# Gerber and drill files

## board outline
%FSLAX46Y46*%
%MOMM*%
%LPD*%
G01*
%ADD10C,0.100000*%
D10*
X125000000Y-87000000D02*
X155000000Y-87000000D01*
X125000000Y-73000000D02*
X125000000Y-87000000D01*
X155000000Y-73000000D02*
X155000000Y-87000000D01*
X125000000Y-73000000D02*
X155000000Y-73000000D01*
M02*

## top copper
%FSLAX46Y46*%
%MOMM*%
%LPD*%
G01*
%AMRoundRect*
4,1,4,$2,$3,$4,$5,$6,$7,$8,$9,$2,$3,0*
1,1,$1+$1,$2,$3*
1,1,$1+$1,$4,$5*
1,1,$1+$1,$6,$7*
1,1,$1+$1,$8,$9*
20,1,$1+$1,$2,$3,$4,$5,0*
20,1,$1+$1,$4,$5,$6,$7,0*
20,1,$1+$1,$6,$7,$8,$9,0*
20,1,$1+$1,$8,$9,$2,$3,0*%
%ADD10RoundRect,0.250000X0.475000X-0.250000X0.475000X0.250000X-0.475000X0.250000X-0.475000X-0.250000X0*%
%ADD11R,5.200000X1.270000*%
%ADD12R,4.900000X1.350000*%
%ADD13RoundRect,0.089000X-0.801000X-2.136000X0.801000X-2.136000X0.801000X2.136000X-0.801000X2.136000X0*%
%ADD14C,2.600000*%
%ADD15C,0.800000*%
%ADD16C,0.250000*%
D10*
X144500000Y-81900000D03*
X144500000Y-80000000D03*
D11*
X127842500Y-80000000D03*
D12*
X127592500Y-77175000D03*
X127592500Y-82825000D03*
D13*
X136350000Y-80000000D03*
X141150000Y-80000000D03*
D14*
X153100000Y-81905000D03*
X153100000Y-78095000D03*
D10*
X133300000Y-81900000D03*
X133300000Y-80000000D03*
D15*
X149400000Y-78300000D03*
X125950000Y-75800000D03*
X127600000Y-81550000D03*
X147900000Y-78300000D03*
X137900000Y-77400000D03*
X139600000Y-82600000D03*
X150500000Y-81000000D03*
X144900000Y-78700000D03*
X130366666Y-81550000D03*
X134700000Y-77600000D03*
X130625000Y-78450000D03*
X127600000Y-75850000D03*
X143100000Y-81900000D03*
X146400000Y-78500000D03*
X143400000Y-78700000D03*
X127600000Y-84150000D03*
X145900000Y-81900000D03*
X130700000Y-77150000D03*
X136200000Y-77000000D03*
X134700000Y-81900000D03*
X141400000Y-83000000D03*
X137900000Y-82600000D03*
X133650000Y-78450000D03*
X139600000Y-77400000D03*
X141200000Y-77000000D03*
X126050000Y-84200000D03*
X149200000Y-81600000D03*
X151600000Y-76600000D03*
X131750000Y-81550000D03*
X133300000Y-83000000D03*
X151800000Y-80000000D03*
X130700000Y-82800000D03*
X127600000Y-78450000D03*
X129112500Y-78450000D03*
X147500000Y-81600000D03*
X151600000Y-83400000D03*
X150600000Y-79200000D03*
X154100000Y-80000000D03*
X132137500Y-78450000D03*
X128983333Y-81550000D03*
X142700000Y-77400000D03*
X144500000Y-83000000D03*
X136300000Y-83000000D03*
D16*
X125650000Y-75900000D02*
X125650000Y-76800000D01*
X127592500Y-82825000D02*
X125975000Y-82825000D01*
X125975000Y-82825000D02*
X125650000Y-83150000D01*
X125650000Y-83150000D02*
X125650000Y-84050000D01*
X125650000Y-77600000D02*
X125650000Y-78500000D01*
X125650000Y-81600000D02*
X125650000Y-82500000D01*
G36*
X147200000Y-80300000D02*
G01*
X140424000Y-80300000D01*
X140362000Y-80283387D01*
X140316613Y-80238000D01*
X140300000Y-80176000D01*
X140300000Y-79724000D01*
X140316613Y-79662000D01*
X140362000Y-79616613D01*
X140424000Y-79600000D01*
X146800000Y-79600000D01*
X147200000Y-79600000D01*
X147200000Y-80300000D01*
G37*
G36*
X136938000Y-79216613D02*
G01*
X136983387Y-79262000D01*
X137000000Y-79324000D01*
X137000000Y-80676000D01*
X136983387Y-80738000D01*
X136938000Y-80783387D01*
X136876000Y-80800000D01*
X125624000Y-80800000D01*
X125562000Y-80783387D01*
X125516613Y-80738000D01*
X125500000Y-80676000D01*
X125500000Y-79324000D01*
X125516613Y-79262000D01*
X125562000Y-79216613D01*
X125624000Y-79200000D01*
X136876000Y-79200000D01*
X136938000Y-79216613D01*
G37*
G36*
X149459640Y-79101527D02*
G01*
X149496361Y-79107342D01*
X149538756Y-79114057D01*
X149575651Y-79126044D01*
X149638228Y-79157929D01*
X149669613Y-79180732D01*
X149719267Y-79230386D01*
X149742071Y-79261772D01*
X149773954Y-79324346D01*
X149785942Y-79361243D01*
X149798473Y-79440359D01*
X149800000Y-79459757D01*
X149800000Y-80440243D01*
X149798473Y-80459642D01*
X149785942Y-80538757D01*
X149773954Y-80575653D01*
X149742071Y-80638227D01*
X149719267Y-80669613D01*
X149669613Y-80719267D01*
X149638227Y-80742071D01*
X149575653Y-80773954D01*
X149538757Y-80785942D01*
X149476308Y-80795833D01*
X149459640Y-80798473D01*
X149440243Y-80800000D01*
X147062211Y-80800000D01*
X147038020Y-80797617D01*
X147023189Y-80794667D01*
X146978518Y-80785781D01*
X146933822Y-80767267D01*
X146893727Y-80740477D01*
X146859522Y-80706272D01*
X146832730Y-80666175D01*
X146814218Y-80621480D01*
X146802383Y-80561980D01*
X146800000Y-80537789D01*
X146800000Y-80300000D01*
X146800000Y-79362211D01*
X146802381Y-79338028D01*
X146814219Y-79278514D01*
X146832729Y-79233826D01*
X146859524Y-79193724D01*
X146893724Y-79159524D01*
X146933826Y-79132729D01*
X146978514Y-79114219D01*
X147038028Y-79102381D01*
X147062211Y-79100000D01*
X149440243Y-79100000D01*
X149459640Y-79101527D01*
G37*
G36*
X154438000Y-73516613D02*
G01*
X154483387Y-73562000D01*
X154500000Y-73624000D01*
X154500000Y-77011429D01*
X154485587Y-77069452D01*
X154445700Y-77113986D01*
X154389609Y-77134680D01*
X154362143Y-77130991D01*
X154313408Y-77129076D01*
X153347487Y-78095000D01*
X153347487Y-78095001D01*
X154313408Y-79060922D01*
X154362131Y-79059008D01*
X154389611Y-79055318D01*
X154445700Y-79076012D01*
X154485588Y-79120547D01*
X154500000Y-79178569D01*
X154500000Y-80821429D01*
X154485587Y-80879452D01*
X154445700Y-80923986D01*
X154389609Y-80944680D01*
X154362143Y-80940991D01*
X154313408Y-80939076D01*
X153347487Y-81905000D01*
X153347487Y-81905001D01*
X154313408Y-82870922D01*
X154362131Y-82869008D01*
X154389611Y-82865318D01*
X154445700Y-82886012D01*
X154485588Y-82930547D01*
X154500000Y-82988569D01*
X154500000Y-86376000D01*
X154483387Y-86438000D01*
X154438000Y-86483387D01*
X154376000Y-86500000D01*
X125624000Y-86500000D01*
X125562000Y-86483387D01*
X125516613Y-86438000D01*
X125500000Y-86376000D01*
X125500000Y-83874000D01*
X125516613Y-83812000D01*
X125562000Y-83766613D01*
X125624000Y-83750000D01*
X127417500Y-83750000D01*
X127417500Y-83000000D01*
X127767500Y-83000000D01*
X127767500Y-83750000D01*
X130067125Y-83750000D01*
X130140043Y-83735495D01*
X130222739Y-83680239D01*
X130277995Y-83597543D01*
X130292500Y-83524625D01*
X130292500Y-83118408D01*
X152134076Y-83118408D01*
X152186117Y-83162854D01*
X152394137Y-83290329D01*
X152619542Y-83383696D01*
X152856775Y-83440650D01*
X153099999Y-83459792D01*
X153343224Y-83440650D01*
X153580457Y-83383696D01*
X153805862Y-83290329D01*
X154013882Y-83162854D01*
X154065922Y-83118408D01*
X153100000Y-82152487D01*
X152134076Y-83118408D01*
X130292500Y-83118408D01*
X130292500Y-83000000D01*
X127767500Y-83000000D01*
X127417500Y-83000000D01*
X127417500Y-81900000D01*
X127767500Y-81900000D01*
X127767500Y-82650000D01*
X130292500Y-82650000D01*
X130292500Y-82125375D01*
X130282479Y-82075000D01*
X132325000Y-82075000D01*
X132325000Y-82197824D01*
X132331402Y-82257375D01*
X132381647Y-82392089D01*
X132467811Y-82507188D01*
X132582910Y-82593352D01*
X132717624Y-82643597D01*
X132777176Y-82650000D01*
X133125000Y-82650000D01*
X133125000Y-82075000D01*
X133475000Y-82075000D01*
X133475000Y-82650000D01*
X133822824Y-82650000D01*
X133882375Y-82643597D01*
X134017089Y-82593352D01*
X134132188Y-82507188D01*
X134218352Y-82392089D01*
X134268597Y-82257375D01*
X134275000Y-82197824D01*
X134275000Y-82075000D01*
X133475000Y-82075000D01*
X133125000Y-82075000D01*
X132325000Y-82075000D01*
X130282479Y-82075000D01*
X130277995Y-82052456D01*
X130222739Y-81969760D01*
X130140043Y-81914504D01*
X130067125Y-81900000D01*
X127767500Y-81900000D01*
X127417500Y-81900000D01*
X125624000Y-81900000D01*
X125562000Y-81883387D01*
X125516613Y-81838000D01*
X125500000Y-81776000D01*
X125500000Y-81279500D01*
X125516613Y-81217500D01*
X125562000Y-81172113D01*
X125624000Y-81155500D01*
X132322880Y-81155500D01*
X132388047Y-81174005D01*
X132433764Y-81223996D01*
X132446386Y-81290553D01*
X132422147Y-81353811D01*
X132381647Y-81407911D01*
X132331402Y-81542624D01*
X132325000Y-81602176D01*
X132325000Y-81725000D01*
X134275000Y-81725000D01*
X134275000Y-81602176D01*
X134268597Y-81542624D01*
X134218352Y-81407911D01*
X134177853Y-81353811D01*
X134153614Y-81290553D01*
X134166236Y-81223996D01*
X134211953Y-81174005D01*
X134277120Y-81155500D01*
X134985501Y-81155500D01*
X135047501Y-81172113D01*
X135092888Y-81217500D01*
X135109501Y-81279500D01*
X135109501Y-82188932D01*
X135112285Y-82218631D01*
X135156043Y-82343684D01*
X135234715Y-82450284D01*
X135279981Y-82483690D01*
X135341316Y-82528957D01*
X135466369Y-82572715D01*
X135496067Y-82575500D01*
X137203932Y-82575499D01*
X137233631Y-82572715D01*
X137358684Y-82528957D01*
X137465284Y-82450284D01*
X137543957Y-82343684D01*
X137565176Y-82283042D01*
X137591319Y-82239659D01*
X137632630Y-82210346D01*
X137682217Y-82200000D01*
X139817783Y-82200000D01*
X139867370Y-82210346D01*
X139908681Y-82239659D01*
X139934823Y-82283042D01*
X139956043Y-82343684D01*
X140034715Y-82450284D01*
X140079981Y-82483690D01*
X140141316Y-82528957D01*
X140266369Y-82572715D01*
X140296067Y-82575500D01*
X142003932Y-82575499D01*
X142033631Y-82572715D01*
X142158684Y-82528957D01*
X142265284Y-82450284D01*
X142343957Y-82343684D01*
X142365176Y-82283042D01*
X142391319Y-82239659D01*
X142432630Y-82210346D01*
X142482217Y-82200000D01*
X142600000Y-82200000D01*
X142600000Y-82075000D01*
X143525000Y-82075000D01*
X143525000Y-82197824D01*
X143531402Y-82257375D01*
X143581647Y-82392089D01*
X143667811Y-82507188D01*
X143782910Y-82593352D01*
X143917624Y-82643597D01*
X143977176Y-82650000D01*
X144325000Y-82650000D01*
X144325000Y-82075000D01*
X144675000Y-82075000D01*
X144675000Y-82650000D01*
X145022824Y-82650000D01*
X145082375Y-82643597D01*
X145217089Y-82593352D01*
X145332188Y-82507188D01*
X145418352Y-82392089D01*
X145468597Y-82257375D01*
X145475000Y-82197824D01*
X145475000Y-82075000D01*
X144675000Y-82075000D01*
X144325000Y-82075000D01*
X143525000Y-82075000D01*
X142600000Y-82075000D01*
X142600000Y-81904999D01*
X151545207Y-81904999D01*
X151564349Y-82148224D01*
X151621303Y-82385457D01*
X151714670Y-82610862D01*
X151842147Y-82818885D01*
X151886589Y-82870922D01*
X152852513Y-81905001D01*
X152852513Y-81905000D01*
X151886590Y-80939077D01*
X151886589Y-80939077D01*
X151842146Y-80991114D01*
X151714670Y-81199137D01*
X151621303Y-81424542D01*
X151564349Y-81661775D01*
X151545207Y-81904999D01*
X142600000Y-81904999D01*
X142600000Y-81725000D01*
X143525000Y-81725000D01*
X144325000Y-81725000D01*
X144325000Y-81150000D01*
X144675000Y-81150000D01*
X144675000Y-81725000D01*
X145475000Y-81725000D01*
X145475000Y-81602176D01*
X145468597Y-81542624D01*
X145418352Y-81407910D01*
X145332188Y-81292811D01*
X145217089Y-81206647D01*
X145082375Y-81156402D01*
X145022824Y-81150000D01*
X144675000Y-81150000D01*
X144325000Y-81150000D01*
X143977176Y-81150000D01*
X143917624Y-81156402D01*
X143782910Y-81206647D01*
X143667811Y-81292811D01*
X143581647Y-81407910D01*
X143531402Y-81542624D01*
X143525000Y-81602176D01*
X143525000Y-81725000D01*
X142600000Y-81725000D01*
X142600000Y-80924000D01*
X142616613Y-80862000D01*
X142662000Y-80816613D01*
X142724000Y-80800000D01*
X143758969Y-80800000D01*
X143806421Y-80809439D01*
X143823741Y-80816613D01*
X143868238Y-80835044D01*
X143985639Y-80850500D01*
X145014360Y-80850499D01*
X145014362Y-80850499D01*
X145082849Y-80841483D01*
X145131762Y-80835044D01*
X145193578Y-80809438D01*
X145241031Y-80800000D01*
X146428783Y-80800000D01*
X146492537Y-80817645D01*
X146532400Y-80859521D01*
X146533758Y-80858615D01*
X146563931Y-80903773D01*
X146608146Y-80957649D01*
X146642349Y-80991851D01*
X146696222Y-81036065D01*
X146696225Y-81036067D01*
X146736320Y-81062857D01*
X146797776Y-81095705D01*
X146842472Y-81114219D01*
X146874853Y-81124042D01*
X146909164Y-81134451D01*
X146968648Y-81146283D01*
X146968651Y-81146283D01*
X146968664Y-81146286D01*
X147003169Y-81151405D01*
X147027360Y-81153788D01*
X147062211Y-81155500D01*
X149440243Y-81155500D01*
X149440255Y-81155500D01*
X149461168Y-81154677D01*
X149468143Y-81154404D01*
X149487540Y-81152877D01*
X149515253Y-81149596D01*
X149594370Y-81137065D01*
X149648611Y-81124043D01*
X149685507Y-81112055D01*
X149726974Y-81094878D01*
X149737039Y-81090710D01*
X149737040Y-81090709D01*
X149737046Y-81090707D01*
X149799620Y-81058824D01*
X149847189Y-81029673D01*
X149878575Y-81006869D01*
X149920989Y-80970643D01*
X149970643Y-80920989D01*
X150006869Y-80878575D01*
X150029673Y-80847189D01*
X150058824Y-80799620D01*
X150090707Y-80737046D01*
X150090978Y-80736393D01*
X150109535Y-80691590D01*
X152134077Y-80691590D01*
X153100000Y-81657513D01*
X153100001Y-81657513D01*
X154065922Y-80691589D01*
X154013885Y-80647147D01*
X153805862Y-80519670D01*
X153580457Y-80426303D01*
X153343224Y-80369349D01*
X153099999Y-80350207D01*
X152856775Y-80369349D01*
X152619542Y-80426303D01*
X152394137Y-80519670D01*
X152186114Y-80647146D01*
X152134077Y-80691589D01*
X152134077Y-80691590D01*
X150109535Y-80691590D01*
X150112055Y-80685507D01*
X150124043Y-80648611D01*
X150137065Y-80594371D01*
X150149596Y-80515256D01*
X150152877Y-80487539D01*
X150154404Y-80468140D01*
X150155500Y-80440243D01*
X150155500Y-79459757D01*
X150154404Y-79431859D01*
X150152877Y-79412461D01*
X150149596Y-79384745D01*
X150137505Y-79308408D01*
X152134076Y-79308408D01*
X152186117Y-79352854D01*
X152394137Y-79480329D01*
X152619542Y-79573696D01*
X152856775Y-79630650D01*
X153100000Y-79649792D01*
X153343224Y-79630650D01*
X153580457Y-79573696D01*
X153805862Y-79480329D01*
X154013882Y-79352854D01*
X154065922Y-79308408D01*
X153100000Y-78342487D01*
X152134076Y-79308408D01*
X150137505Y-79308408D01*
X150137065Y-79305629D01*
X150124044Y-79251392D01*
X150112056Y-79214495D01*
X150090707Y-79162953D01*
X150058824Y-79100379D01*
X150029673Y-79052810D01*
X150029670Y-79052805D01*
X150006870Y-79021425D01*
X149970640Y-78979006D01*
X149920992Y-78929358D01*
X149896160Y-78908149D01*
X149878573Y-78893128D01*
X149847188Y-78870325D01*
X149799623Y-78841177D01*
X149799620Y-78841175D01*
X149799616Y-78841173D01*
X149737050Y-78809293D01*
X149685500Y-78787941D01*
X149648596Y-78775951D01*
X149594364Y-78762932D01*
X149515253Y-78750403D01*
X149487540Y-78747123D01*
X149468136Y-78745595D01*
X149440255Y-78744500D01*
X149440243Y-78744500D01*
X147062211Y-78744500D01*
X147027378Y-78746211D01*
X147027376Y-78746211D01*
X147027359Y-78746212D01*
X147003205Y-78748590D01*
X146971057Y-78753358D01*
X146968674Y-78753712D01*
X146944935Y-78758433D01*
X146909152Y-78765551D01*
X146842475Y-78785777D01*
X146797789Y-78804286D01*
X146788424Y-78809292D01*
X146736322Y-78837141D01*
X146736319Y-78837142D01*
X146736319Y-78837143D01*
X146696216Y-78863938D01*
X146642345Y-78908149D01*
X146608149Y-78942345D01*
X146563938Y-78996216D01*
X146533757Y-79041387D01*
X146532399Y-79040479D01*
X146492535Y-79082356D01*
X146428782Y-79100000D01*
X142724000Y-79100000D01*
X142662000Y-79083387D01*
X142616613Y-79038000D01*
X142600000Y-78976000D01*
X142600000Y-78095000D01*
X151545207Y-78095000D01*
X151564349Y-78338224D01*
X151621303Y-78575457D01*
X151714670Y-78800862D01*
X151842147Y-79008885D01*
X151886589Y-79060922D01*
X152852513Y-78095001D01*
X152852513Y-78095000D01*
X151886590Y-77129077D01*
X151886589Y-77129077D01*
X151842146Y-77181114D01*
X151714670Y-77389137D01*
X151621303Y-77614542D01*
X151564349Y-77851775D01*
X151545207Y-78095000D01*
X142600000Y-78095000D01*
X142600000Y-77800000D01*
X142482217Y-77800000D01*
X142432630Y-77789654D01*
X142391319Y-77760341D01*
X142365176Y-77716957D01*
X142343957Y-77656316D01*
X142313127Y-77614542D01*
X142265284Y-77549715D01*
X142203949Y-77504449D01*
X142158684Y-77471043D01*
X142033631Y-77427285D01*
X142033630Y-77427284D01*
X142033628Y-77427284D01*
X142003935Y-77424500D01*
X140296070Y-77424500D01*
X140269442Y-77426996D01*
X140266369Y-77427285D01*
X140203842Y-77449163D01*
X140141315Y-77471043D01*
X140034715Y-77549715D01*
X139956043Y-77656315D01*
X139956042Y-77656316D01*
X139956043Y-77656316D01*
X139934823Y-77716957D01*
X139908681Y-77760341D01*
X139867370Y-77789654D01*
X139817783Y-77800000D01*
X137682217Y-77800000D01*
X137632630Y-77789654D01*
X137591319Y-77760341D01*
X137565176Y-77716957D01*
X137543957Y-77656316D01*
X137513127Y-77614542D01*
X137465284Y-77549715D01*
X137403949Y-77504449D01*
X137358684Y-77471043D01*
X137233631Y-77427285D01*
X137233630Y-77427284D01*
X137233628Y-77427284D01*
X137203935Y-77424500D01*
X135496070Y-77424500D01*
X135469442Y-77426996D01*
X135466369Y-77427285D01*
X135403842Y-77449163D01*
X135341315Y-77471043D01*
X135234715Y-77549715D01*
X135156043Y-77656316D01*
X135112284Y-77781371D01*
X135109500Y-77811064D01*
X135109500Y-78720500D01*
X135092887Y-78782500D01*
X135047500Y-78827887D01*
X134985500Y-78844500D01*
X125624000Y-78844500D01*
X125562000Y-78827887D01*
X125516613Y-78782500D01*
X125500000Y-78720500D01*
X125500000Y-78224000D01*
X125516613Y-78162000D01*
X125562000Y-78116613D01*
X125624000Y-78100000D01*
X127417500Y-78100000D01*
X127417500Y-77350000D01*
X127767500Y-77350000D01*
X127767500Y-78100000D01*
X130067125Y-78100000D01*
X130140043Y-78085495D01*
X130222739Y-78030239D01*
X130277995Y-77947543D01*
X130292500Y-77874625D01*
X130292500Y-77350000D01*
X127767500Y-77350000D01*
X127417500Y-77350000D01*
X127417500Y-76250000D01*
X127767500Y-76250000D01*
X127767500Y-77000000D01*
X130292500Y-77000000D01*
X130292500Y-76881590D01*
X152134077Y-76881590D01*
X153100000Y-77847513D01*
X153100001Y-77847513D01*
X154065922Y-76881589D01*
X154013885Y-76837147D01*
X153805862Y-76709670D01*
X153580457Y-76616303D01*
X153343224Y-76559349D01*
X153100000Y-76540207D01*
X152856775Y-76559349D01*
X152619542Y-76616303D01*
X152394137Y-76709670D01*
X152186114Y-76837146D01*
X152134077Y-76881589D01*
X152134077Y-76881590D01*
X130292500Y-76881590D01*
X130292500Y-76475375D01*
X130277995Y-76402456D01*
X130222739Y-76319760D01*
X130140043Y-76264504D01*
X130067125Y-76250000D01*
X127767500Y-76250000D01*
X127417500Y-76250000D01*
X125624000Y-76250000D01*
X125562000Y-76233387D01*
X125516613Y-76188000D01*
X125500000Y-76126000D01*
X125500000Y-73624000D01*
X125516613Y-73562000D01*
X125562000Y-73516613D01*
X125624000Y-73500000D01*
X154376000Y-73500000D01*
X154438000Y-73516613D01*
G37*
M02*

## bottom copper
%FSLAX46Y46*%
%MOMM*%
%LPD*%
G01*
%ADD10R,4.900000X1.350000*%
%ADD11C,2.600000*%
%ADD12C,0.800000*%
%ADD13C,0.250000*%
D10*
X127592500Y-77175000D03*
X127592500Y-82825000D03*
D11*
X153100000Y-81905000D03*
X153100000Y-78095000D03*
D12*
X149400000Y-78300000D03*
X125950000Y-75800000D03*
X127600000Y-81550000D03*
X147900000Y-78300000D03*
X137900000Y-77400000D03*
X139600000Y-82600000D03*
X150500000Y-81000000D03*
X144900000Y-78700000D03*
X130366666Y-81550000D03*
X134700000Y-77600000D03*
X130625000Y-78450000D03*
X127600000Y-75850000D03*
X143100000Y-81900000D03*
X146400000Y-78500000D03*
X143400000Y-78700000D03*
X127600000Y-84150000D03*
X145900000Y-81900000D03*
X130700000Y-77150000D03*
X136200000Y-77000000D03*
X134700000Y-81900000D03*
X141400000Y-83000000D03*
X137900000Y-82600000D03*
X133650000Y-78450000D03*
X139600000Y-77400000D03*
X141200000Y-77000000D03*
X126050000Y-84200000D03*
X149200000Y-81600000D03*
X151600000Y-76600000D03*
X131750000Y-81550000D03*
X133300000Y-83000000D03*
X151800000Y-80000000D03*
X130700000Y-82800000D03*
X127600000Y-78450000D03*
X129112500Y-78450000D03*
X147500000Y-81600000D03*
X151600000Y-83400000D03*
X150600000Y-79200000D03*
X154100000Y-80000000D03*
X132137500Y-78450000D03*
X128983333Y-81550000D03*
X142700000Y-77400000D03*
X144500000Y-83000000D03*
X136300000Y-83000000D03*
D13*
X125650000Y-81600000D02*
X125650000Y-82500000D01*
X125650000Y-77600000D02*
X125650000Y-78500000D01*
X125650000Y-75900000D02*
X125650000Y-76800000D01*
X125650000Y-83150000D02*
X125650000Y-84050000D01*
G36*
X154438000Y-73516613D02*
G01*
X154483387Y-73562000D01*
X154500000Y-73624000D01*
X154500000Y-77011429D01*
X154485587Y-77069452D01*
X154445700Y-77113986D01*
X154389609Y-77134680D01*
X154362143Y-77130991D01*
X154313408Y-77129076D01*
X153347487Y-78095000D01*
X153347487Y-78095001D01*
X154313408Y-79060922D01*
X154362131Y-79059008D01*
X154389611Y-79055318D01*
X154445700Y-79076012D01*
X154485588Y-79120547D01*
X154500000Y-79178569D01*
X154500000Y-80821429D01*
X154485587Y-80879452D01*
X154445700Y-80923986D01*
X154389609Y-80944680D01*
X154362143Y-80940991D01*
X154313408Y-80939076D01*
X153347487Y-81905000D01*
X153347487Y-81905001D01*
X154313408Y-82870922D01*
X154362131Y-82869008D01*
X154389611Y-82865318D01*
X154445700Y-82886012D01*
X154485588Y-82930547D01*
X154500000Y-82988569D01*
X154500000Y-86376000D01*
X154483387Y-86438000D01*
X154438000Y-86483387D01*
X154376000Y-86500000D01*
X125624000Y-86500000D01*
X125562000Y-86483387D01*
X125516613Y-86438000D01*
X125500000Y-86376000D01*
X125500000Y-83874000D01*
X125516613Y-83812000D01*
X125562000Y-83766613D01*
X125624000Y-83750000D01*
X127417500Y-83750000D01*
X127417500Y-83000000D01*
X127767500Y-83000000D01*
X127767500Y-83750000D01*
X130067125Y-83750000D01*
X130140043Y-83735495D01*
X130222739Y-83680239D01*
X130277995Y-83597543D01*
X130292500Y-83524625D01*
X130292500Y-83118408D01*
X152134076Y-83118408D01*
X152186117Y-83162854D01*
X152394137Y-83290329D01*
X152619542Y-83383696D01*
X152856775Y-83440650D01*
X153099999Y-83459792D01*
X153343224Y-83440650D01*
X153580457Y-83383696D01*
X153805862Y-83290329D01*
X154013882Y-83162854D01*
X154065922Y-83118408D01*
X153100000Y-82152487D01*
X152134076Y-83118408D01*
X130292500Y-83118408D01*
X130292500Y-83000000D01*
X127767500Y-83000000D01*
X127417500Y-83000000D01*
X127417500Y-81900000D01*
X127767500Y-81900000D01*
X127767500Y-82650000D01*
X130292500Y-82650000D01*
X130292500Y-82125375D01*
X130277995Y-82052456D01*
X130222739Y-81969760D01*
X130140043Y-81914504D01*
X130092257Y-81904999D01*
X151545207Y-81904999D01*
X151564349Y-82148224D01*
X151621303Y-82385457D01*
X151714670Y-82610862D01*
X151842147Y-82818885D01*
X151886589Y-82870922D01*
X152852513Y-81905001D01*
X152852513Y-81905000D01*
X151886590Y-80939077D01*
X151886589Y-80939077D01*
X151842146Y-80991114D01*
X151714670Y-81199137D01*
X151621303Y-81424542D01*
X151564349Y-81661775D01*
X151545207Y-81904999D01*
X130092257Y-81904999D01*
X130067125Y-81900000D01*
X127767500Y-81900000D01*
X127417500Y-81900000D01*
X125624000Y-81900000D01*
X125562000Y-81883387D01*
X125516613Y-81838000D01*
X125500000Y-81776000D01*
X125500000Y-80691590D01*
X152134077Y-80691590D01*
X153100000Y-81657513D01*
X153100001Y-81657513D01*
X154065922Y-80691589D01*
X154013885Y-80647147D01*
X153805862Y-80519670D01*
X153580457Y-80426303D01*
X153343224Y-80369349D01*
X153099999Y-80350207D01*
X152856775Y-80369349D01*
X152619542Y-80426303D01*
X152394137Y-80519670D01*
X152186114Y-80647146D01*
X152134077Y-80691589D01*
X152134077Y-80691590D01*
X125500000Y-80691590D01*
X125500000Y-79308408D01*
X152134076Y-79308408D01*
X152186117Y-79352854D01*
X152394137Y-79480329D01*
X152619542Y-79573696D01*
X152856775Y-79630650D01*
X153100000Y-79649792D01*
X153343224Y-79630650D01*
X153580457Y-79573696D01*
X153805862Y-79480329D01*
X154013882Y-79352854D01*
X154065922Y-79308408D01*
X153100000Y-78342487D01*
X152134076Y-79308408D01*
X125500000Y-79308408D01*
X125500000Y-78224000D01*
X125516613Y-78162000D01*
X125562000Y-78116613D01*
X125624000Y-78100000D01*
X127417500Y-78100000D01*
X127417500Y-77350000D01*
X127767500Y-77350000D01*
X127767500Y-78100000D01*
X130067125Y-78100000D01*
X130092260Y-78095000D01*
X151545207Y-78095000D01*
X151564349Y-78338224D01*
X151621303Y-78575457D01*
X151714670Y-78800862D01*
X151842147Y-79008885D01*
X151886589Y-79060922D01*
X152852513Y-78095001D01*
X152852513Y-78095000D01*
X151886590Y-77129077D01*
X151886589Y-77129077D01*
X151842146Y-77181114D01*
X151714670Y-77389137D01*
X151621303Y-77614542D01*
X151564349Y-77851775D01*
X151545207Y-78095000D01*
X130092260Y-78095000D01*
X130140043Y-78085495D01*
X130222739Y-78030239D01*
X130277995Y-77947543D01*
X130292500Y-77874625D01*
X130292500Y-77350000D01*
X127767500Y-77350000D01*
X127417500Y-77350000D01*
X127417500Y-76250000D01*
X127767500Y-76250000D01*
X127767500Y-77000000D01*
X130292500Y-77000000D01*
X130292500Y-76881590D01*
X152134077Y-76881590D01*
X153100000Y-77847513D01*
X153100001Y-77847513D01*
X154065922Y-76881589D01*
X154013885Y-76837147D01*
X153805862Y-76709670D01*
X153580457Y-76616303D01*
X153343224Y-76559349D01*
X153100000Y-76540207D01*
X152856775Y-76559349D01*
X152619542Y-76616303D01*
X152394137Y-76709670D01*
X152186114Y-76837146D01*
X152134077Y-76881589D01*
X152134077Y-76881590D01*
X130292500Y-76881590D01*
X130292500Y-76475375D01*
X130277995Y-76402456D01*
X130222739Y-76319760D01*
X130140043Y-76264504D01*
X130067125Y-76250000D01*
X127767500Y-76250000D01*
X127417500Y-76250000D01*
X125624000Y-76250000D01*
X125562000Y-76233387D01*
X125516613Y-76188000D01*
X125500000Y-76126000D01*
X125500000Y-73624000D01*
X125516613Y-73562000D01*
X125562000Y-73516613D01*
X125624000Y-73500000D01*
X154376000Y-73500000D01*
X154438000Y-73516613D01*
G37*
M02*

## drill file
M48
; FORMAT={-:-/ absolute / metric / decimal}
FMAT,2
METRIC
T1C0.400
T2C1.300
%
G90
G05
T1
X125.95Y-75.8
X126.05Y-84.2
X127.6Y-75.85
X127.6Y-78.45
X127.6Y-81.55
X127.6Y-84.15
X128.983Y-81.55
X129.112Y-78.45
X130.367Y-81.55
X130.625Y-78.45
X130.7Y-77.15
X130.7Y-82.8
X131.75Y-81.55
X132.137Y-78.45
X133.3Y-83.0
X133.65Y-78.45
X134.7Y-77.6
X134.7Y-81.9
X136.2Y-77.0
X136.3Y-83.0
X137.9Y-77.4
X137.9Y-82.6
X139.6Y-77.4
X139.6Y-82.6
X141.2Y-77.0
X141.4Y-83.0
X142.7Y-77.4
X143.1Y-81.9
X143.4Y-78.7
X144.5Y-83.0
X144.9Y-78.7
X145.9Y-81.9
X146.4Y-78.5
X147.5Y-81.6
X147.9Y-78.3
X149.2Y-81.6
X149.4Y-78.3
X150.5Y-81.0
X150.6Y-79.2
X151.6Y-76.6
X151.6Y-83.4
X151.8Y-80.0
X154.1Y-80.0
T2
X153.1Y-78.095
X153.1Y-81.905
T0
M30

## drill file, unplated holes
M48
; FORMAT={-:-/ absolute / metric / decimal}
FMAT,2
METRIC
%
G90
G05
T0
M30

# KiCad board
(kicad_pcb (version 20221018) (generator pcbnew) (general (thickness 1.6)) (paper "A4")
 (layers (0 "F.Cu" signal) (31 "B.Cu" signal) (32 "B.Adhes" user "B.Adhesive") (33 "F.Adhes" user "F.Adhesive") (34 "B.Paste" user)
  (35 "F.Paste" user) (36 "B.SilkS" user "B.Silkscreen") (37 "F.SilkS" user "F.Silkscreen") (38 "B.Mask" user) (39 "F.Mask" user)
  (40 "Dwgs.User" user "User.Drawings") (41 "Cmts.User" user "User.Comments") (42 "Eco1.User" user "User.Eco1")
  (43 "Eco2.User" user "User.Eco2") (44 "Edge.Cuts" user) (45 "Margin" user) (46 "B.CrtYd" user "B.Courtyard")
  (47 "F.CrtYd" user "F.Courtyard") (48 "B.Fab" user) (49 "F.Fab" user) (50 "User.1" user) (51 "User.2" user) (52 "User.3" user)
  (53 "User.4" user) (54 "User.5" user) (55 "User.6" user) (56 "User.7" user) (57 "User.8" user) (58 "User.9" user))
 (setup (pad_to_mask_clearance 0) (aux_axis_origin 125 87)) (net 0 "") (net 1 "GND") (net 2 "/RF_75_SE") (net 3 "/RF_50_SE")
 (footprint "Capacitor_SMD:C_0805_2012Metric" (layer "F.Cu") (at 144.5 80.95 90)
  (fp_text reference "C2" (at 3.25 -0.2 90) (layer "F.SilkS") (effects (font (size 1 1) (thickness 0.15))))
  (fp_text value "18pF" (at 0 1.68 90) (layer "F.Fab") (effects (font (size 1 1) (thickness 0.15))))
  (pad "1" smd roundrect (at -0.95 0 90) (size 1 1.45) (layers "F.Cu" "F.Paste" "F.Mask") (roundrect_rratio 0.25) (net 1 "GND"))
  (pad "2" smd roundrect (at 0.95 0 90) (size 1 1.45) (layers "F.Cu" "F.Paste" "F.Mask") (roundrect_rratio 0.25) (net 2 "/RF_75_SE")))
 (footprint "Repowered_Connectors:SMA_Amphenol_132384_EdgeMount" (layer "F.Cu") (at 127.2425 80 -90) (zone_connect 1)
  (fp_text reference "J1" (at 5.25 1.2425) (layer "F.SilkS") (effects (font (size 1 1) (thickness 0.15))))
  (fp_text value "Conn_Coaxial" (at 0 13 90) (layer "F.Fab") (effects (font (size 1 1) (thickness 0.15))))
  (pad "1" smd rect (at 0 -0.6 270) (size 1.27 5.2) (layers "F.Cu" "F.Paste" "F.Mask") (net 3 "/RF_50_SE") (zone_connect 2))
  (pad "2" smd rect (at -2.825 -0.35 270) (size 1.35 4.9) (layers "F.Cu" "F.Paste" "F.Mask") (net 1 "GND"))
  (pad "2" smd rect (at -2.825 -0.35 270) (size 1.35 4.9) (layers "B.Cu" "B.Paste" "B.Mask") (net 1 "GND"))
  (pad "2" smd rect (at 2.825 -0.35 270) (size 1.35 4.9) (layers "F.Cu" "F.Paste" "F.Mask") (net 1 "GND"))
  (pad "2" smd rect (at 2.825 -0.35 270) (size 1.35 4.9) (layers "B.Cu" "B.Paste" "B.Mask") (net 1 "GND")))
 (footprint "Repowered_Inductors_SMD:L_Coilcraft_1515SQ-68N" (layer "F.Cu") (at 138.75 80)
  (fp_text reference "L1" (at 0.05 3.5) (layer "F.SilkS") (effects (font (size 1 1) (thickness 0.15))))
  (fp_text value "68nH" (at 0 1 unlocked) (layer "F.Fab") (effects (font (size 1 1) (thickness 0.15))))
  (pad "1" smd roundrect (at -2.4 0) (size 1.78 4.45) (layers "F.Cu" "F.Paste" "F.Mask") (roundrect_rratio 0.05) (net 3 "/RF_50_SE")
   (thermal_bridge_angle 45))
  (pad "2" smd roundrect (at 2.4 0) (size 1.78 4.45) (layers "F.Cu" "F.Paste" "F.Mask") (roundrect_rratio 0.05) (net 2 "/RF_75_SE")
   (thermal_bridge_angle 45)))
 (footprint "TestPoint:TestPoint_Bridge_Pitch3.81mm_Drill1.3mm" (layer "F.Cu") (at 153.1 81.905 90)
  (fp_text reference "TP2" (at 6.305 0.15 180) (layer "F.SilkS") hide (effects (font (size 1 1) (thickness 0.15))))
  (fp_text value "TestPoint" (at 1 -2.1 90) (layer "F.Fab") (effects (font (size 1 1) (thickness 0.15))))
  (pad "1" thru_hole circle (at 0 0 90) (size 2.6 2.6) (drill 1.3) (layers "*.Cu" "*.Mask") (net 1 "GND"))
  (pad "1" thru_hole circle (at 3.81 0 90) (size 2.6 2.6) (drill 1.3) (layers "*.Cu" "*.Mask") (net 1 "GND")))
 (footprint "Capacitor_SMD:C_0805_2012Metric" (layer "F.Cu") (at 133.3 80.95 90)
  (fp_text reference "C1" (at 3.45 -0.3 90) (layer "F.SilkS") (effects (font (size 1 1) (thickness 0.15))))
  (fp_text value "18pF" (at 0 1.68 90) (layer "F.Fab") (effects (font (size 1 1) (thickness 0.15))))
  (pad "1" smd roundrect (at -0.95 0 90) (size 1 1.45) (layers "F.Cu" "F.Paste" "F.Mask") (roundrect_rratio 0.25) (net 1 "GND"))
  (pad "2" smd roundrect (at 0.95 0 90) (size 1 1.45) (layers "F.Cu" "F.Paste" "F.Mask") (roundrect_rratio 0.25) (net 3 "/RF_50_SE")))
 (gr_line (start 125 87) (end 155 87) (stroke (width 0.1) (type default)) (layer "Edge.Cuts"))
 (gr_line (start 125 73) (end 125 87) (stroke (width 0.1) (type default)) (layer "Edge.Cuts"))
 (gr_line (start 155 73) (end 155 87) (stroke (width 0.1) (type default)) (layer "Edge.Cuts"))
 (gr_line (start 125 73) (end 155 73) (stroke (width 0.1) (type default)) (layer "Edge.Cuts"))
 (segment (start 125.65 75.9) (end 125.65 76.8) (width 0.25) (layer "F.Cu") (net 1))
 (segment (start 127.5925 82.825) (end 125.975 82.825) (width 0.25) (layer "F.Cu") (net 1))
 (segment (start 125.975 82.825) (end 125.65 83.15) (width 0.25) (layer "F.Cu") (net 1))
 (segment (start 125.65 83.15) (end 125.65 84.05) (width 0.25) (layer "F.Cu") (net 1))
 (segment (start 125.65 77.6) (end 125.65 78.5) (width 0.25) (layer "F.Cu") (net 1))
 (segment (start 125.65 81.6) (end 125.65 82.5) (width 0.25) (layer "F.Cu") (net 1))
 (via (at 149.4 78.3) (size 0.8) (drill 0.4) (layers "F.Cu" "B.Cu") (free) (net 1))
 (via (at 125.95 75.8) (size 0.8) (drill 0.4) (layers "F.Cu" "B.Cu") (free) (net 1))
 (via (at 127.6 81.55) (size 0.8) (drill 0.4) (layers "F.Cu" "B.Cu") (free) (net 1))
 (via (at 147.9 78.3) (size 0.8) (drill 0.4) (layers "F.Cu" "B.Cu") (free) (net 1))
 (via (at 137.9 77.4) (size 0.8) (drill 0.4) (layers "F.Cu" "B.Cu") (free) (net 1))
 (via (at 139.6 82.6) (size 0.8) (drill 0.4) (layers "F.Cu" "B.Cu") (free) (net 1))
 (via (at 150.5 81) (size 0.8) (drill 0.4) (layers "F.Cu" "B.Cu") (free) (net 1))
 (via (at 144.9 78.7) (size 0.8) (drill 0.4) (layers "F.Cu" "B.Cu") (free) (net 1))
 (via (at 130.366666 81.55) (size 0.8) (drill 0.4) (layers "F.Cu" "B.Cu") (free) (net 1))
 (via (at 134.7 77.6) (size 0.8) (drill 0.4) (layers "F.Cu" "B.Cu") (free) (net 1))
 (via (at 130.625 78.45) (size 0.8) (drill 0.4) (layers "F.Cu" "B.Cu") (free) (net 1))
 (via (at 127.6 75.85) (size 0.8) (drill 0.4) (layers "F.Cu" "B.Cu") (free) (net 1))
 (via (at 143.1 81.9) (size 0.8) (drill 0.4) (layers "F.Cu" "B.Cu") (free) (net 1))
 (via (at 146.4 78.5) (size 0.8) (drill 0.4) (layers "F.Cu" "B.Cu") (free) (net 1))
 (via (at 143.4 78.7) (size 0.8) (drill 0.4) (layers "F.Cu" "B.Cu") (free) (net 1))
 (via (at 127.6 84.15) (size 0.8) (drill 0.4) (layers "F.Cu" "B.Cu") (free) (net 1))
 (via (at 145.9 81.9) (size 0.8) (drill 0.4) (layers "F.Cu" "B.Cu") (free) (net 1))
 (via (at 130.7 77.15) (size 0.8) (drill 0.4) (layers "F.Cu" "B.Cu") (free) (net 1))
 (via (at 136.2 77) (size 0.8) (drill 0.4) (layers "F.Cu" "B.Cu") (free) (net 1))
 (via (at 134.7 81.9) (size 0.8) (drill 0.4) (layers "F.Cu" "B.Cu") (free) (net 1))
 (via (at 141.4 83) (size 0.8) (drill 0.4) (layers "F.Cu" "B.Cu") (free) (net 1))
 (via (at 137.9 82.6) (size 0.8) (drill 0.4) (layers "F.Cu" "B.Cu") (free) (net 1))
 (via (at 133.65 78.45) (size 0.8) (drill 0.4) (layers "F.Cu" "B.Cu") (free) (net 1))
 (via (at 139.6 77.4) (size 0.8) (drill 0.4) (layers "F.Cu" "B.Cu") (free) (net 1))
 (via (at 141.2 77) (size 0.8) (drill 0.4) (layers "F.Cu" "B.Cu") (free) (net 1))
 (via (at 126.05 84.2) (size 0.8) (drill 0.4) (layers "F.Cu" "B.Cu") (free) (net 1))
 (via (at 149.2 81.6) (size 0.8) (drill 0.4) (layers "F.Cu" "B.Cu") (free) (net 1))
 (via (at 151.6 76.6) (size 0.8) (drill 0.4) (layers "F.Cu" "B.Cu") (free) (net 1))
 (via (at 131.75 81.55) (size 0.8) (drill 0.4) (layers "F.Cu" "B.Cu") (free) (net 1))
 (via (at 133.3 83) (size 0.8) (drill 0.4) (layers "F.Cu" "B.Cu") (free) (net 1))
 (via (at 151.8 80) (size 0.8) (drill 0.4) (layers "F.Cu" "B.Cu") (free) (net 1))
 (via (at 130.7 82.8) (size 0.8) (drill 0.4) (layers "F.Cu" "B.Cu") (free) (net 1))
 (via (at 127.6 78.45) (size 0.8) (drill 0.4) (layers "F.Cu" "B.Cu") (free) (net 1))
 (via (at 129.1125 78.45) (size 0.8) (drill 0.4) (layers "F.Cu" "B.Cu") (free) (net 1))
 (via (at 147.5 81.6) (size 0.8) (drill 0.4) (layers "F.Cu" "B.Cu") (free) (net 1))
 (via (at 151.6 83.4) (size 0.8) (drill 0.4) (layers "F.Cu" "B.Cu") (free) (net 1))
 (via (at 150.6 79.2) (size 0.8) (drill 0.4) (layers "F.Cu" "B.Cu") (free) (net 1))
 (via (at 154.1 80) (size 0.8) (drill 0.4) (layers "F.Cu" "B.Cu") (free) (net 1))
 (via (at 132.1375 78.45) (size 0.8) (drill 0.4) (layers "F.Cu" "B.Cu") (free) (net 1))
 (via (at 128.983333 81.55) (size 0.8) (drill 0.4) (layers "F.Cu" "B.Cu") (free) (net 1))
 (via (at 142.7 77.4) (size 0.8) (drill 0.4) (layers "F.Cu" "B.Cu") (free) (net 1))
 (via (at 144.5 83) (size 0.8) (drill 0.4) (layers "F.Cu" "B.Cu") (free) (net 1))
 (via (at 136.3 83) (size 0.8) (drill 0.4) (layers "F.Cu" "B.Cu") (free) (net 1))
 (segment (start 125.65 81.6) (end 125.65 82.5) (width 0.25) (layer "B.Cu") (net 1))
 (segment (start 125.65 77.6) (end 125.65 78.5) (width 0.25) (layer "B.Cu") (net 1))
 (segment (start 125.65 75.9) (end 125.65 76.8) (width 0.25) (layer "B.Cu") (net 1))
 (segment (start 125.65 83.15) (end 125.65 84.05) (width 0.25) (layer "B.Cu") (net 1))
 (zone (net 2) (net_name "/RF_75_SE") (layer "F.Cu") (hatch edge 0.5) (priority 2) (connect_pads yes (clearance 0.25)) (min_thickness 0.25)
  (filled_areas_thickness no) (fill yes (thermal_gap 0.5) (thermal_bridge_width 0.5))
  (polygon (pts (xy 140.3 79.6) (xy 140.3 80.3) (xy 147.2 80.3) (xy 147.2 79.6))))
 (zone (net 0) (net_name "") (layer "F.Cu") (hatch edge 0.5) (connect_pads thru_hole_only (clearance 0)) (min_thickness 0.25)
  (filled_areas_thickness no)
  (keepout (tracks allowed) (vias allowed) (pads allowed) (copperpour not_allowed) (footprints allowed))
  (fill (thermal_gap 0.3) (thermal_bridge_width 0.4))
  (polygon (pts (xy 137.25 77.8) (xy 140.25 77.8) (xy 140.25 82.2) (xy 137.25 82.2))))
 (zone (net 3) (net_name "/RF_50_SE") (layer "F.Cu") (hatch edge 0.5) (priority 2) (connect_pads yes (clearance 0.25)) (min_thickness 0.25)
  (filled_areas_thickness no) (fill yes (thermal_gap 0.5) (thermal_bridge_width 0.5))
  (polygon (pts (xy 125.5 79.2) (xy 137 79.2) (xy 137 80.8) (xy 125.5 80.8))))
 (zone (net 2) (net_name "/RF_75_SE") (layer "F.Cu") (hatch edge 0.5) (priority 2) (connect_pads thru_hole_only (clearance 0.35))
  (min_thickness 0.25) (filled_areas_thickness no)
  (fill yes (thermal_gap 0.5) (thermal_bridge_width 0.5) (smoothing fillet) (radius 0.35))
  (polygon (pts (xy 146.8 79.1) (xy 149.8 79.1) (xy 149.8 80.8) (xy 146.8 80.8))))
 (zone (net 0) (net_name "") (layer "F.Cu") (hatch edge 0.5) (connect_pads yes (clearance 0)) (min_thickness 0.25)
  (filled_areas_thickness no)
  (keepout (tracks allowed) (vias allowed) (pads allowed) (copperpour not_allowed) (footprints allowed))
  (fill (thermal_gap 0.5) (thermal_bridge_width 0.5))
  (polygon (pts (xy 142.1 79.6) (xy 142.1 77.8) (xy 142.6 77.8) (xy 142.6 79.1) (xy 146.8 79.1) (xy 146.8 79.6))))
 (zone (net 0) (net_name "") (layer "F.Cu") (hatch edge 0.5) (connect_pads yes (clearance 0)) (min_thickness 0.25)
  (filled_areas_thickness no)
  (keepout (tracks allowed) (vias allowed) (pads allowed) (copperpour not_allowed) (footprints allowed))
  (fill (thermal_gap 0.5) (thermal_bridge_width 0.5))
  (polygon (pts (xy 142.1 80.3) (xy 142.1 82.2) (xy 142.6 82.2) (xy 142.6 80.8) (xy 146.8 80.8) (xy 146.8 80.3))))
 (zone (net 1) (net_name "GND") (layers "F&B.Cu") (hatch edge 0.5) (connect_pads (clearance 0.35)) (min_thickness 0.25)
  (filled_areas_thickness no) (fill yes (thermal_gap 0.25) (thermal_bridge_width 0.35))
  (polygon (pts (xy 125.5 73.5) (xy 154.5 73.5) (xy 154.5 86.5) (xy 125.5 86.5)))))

